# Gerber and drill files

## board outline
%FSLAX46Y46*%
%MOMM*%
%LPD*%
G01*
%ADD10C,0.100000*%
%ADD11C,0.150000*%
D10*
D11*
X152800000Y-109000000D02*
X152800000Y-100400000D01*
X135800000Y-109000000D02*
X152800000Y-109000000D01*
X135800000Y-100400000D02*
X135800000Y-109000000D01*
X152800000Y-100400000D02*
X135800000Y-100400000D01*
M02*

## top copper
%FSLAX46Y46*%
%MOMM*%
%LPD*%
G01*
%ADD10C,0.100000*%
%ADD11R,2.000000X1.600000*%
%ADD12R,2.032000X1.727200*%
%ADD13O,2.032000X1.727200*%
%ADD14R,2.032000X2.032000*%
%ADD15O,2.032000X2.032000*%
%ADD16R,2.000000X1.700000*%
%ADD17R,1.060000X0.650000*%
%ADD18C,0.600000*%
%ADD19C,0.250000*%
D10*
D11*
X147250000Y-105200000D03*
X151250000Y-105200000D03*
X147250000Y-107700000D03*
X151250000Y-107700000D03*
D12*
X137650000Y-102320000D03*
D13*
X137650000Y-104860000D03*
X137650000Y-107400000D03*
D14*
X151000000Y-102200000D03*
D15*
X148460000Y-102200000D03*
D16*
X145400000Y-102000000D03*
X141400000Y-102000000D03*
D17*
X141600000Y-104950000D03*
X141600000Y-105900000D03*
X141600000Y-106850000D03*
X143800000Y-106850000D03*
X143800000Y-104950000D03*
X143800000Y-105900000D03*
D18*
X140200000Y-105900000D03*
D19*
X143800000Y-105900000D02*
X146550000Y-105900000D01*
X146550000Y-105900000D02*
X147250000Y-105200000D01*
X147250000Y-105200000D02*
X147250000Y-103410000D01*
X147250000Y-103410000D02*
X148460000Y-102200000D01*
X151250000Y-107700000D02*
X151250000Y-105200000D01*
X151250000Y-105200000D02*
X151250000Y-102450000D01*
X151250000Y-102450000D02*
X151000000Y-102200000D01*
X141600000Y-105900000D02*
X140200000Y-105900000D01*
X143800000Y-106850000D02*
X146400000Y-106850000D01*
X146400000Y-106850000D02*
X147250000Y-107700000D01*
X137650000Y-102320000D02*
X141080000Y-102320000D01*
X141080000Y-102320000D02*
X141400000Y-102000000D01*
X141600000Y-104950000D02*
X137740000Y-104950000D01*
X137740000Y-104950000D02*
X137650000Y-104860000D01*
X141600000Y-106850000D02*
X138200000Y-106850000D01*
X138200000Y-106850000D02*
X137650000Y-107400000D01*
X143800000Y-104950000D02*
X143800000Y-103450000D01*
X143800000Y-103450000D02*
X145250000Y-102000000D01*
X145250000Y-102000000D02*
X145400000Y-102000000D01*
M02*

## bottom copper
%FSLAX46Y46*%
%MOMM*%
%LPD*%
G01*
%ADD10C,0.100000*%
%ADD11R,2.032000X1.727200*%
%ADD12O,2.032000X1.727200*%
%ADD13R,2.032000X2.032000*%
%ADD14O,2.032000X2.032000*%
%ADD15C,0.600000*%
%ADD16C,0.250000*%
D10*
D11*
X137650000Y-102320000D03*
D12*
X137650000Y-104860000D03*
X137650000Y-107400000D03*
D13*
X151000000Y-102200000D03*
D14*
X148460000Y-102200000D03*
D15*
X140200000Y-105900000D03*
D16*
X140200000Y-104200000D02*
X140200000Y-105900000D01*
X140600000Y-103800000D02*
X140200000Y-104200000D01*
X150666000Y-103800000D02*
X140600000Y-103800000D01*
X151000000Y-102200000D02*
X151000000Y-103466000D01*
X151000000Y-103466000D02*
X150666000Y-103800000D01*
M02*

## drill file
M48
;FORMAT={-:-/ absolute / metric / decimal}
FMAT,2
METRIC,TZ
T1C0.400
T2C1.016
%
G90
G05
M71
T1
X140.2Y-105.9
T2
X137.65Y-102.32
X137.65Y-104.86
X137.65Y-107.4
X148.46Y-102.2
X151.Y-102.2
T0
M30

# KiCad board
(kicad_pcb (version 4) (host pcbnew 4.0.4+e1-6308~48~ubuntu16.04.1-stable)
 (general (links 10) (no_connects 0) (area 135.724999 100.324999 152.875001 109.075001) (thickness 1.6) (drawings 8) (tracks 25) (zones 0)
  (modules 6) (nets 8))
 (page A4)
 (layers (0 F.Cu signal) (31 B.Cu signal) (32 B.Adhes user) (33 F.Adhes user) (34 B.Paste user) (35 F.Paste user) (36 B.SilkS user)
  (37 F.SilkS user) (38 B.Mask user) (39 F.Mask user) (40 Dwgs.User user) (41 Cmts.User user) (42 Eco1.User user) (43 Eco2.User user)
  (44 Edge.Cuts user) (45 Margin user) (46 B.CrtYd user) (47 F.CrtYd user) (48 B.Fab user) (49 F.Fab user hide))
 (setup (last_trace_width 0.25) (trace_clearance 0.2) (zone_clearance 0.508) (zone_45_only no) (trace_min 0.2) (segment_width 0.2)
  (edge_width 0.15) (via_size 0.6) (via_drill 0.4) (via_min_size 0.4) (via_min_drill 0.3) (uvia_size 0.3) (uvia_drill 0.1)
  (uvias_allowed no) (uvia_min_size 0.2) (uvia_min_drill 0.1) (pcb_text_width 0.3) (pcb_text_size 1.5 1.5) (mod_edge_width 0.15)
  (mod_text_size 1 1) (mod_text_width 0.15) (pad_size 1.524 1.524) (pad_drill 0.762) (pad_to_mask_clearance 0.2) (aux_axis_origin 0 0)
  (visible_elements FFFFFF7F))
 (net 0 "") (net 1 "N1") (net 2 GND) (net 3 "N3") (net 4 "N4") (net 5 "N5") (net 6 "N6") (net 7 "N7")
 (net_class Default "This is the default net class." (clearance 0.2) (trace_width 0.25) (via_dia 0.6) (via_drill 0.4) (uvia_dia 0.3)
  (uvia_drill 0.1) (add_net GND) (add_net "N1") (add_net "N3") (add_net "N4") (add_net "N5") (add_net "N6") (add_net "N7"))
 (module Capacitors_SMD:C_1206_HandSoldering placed (layer F.Cu) (at 149.25 105.2)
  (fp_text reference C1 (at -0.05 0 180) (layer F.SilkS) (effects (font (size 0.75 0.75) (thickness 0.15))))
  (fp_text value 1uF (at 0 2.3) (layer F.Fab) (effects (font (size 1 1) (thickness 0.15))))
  (pad 1 smd rect (at -2 0) (size 2 1.6) (layers F.Cu F.Paste F.Mask) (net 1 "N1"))
  (pad 2 smd rect (at 2 0) (size 2 1.6) (layers F.Cu F.Paste F.Mask) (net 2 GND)))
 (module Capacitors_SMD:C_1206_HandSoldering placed (layer F.Cu) (at 149.25 107.7)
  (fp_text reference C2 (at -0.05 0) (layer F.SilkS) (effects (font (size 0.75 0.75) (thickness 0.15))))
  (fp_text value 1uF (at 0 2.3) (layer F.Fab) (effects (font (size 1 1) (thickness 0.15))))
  (pad 1 smd rect (at -2 0) (size 2 1.6) (layers F.Cu F.Paste F.Mask) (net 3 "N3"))
  (pad 2 smd rect (at 2 0) (size 2 1.6) (layers F.Cu F.Paste F.Mask) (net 2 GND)))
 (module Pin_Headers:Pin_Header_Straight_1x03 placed (layer F.Cu) (at 137.65 102.32)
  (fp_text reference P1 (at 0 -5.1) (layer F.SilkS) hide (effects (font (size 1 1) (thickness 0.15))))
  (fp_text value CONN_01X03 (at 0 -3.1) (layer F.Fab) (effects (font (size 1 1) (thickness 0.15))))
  (pad 1 thru_hole rect (at 0 0) (size 2.032 1.7272) (drill 1.016) (layers *.Cu *.Mask F.SilkS) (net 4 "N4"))
  (pad 2 thru_hole oval (at 0 2.54) (size 2.032 1.7272) (drill 1.016) (layers *.Cu *.Mask F.SilkS) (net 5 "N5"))
  (pad 3 thru_hole oval (at 0 5.08) (size 2.032 1.7272) (drill 1.016) (layers *.Cu *.Mask F.SilkS) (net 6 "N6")))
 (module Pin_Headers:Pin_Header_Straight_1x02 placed (layer F.Cu) (at 151 102.2 270)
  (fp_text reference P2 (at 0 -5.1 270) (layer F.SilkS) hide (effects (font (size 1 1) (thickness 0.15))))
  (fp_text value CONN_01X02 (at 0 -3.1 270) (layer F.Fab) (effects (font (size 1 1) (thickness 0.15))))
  (pad 1 thru_hole rect (at 0 0 270) (size 2.032 2.032) (drill 1.016) (layers *.Cu *.Mask F.SilkS) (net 2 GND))
  (pad 2 thru_hole oval (at 0 2.54 270) (size 2.032 2.032) (drill 1.016) (layers *.Cu *.Mask F.SilkS) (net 1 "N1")))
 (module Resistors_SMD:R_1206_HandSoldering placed (layer F.Cu) (at 143.4 102 180)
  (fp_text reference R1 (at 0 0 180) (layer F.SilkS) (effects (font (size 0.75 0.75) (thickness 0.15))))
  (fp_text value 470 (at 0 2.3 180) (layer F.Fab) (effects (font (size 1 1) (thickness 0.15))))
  (pad 1 smd rect (at -2 0 180) (size 2 1.7) (layers F.Cu F.Paste F.Mask) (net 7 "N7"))
  (pad 2 smd rect (at 2 0 180) (size 2 1.7) (layers F.Cu F.Paste F.Mask) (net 4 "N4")))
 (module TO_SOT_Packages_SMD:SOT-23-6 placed (layer F.Cu) (at 142.7 105.9)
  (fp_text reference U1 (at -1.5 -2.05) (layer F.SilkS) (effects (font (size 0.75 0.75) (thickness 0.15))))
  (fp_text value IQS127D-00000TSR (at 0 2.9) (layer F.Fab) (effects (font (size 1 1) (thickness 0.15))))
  (pad 1 smd rect (at -1.1 -0.95) (size 1.06 0.65) (layers F.Cu F.Paste F.Mask) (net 5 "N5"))
  (pad 2 smd rect (at -1.1 0) (size 1.06 0.65) (layers F.Cu F.Paste F.Mask) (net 2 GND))
  (pad 3 smd rect (at -1.1 0.95) (size 1.06 0.65) (layers F.Cu F.Paste F.Mask) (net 6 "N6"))
  (pad 4 smd rect (at 1.1 0.95) (size 1.06 0.65) (layers F.Cu F.Paste F.Mask) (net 3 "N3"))
  (pad 6 smd rect (at 1.1 -0.95) (size 1.06 0.65) (layers F.Cu F.Paste F.Mask) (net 7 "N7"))
  (pad 5 smd rect (at 1.1 0) (size 1.06 0.65) (layers F.Cu F.Paste F.Mask) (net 1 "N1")))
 (gr_line (start 152.8 109) (end 152.8 100.4) (layer Edge.Cuts) (width 0.15))
 (gr_line (start 135.8 109) (end 152.8 109) (layer Edge.Cuts) (width 0.15))
 (gr_line (start 135.8 100.4) (end 135.8 109) (layer Edge.Cuts) (width 0.15))
 (gr_line (start 152.8 100.4) (end 135.8 100.4) (layer Edge.Cuts) (width 0.15))
 (segment (start 143.8 105.9) (end 146.55 105.9) (width 0.25) (layer F.Cu) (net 1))
 (segment (start 146.55 105.9) (end 147.25 105.2) (width 0.25) (layer F.Cu) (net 1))
 (segment (start 147.25 105.2) (end 147.25 103.41) (width 0.25) (layer F.Cu) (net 1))
 (segment (start 147.25 103.41) (end 148.46 102.2) (width 0.25) (layer F.Cu) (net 1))
 (segment (start 140.2 104.2) (end 140.2 105.9) (width 0.25) (layer B.Cu) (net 2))
 (segment (start 140.6 103.8) (end 140.2 104.2) (width 0.25) (layer B.Cu) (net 2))
 (segment (start 150.666 103.8) (end 140.6 103.8) (width 0.25) (layer B.Cu) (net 2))
 (segment (start 151 102.2) (end 151 103.466) (width 0.25) (layer B.Cu) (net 2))
 (segment (start 151 103.466) (end 150.666 103.8) (width 0.25) (layer B.Cu) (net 2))
 (segment (start 151.25 107.7) (end 151.25 105.2) (width 0.25) (layer F.Cu) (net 2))
 (segment (start 151.25 105.2) (end 151.25 102.45) (width 0.25) (layer F.Cu) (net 2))
 (segment (start 151.25 102.45) (end 151 102.2) (width 0.25) (layer F.Cu) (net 2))
 (segment (start 141.6 105.9) (end 140.2 105.9) (width 0.25) (layer F.Cu) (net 2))
 (via (at 140.2 105.9) (size 0.6) (drill 0.4) (layers F.Cu B.Cu) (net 2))
 (segment (start 143.8 106.85) (end 146.4 106.85) (width 0.25) (layer F.Cu) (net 3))
 (segment (start 146.4 106.85) (end 147.25 107.7) (width 0.25) (layer F.Cu) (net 3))
 (segment (start 137.65 102.32) (end 141.08 102.32) (width 0.25) (layer F.Cu) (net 4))
 (segment (start 141.08 102.32) (end 141.4 102) (width 0.25) (layer F.Cu) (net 4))
 (segment (start 141.6 104.95) (end 137.74 104.95) (width 0.25) (layer F.Cu) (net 5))
 (segment (start 137.74 104.95) (end 137.65 104.86) (width 0.25) (layer F.Cu) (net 5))
 (segment (start 141.6 106.85) (end 138.2 106.85) (width 0.25) (layer F.Cu) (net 6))
 (segment (start 138.2 106.85) (end 137.65 107.4) (width 0.25) (layer F.Cu) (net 6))
 (segment (start 143.8 104.95) (end 143.8 103.45) (width 0.25) (layer F.Cu) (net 7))
 (segment (start 143.8 103.45) (end 145.25 102) (width 0.25) (layer F.Cu) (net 7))
 (segment (start 145.25 102) (end 145.4 102) (width 0.25) (layer F.Cu) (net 7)))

